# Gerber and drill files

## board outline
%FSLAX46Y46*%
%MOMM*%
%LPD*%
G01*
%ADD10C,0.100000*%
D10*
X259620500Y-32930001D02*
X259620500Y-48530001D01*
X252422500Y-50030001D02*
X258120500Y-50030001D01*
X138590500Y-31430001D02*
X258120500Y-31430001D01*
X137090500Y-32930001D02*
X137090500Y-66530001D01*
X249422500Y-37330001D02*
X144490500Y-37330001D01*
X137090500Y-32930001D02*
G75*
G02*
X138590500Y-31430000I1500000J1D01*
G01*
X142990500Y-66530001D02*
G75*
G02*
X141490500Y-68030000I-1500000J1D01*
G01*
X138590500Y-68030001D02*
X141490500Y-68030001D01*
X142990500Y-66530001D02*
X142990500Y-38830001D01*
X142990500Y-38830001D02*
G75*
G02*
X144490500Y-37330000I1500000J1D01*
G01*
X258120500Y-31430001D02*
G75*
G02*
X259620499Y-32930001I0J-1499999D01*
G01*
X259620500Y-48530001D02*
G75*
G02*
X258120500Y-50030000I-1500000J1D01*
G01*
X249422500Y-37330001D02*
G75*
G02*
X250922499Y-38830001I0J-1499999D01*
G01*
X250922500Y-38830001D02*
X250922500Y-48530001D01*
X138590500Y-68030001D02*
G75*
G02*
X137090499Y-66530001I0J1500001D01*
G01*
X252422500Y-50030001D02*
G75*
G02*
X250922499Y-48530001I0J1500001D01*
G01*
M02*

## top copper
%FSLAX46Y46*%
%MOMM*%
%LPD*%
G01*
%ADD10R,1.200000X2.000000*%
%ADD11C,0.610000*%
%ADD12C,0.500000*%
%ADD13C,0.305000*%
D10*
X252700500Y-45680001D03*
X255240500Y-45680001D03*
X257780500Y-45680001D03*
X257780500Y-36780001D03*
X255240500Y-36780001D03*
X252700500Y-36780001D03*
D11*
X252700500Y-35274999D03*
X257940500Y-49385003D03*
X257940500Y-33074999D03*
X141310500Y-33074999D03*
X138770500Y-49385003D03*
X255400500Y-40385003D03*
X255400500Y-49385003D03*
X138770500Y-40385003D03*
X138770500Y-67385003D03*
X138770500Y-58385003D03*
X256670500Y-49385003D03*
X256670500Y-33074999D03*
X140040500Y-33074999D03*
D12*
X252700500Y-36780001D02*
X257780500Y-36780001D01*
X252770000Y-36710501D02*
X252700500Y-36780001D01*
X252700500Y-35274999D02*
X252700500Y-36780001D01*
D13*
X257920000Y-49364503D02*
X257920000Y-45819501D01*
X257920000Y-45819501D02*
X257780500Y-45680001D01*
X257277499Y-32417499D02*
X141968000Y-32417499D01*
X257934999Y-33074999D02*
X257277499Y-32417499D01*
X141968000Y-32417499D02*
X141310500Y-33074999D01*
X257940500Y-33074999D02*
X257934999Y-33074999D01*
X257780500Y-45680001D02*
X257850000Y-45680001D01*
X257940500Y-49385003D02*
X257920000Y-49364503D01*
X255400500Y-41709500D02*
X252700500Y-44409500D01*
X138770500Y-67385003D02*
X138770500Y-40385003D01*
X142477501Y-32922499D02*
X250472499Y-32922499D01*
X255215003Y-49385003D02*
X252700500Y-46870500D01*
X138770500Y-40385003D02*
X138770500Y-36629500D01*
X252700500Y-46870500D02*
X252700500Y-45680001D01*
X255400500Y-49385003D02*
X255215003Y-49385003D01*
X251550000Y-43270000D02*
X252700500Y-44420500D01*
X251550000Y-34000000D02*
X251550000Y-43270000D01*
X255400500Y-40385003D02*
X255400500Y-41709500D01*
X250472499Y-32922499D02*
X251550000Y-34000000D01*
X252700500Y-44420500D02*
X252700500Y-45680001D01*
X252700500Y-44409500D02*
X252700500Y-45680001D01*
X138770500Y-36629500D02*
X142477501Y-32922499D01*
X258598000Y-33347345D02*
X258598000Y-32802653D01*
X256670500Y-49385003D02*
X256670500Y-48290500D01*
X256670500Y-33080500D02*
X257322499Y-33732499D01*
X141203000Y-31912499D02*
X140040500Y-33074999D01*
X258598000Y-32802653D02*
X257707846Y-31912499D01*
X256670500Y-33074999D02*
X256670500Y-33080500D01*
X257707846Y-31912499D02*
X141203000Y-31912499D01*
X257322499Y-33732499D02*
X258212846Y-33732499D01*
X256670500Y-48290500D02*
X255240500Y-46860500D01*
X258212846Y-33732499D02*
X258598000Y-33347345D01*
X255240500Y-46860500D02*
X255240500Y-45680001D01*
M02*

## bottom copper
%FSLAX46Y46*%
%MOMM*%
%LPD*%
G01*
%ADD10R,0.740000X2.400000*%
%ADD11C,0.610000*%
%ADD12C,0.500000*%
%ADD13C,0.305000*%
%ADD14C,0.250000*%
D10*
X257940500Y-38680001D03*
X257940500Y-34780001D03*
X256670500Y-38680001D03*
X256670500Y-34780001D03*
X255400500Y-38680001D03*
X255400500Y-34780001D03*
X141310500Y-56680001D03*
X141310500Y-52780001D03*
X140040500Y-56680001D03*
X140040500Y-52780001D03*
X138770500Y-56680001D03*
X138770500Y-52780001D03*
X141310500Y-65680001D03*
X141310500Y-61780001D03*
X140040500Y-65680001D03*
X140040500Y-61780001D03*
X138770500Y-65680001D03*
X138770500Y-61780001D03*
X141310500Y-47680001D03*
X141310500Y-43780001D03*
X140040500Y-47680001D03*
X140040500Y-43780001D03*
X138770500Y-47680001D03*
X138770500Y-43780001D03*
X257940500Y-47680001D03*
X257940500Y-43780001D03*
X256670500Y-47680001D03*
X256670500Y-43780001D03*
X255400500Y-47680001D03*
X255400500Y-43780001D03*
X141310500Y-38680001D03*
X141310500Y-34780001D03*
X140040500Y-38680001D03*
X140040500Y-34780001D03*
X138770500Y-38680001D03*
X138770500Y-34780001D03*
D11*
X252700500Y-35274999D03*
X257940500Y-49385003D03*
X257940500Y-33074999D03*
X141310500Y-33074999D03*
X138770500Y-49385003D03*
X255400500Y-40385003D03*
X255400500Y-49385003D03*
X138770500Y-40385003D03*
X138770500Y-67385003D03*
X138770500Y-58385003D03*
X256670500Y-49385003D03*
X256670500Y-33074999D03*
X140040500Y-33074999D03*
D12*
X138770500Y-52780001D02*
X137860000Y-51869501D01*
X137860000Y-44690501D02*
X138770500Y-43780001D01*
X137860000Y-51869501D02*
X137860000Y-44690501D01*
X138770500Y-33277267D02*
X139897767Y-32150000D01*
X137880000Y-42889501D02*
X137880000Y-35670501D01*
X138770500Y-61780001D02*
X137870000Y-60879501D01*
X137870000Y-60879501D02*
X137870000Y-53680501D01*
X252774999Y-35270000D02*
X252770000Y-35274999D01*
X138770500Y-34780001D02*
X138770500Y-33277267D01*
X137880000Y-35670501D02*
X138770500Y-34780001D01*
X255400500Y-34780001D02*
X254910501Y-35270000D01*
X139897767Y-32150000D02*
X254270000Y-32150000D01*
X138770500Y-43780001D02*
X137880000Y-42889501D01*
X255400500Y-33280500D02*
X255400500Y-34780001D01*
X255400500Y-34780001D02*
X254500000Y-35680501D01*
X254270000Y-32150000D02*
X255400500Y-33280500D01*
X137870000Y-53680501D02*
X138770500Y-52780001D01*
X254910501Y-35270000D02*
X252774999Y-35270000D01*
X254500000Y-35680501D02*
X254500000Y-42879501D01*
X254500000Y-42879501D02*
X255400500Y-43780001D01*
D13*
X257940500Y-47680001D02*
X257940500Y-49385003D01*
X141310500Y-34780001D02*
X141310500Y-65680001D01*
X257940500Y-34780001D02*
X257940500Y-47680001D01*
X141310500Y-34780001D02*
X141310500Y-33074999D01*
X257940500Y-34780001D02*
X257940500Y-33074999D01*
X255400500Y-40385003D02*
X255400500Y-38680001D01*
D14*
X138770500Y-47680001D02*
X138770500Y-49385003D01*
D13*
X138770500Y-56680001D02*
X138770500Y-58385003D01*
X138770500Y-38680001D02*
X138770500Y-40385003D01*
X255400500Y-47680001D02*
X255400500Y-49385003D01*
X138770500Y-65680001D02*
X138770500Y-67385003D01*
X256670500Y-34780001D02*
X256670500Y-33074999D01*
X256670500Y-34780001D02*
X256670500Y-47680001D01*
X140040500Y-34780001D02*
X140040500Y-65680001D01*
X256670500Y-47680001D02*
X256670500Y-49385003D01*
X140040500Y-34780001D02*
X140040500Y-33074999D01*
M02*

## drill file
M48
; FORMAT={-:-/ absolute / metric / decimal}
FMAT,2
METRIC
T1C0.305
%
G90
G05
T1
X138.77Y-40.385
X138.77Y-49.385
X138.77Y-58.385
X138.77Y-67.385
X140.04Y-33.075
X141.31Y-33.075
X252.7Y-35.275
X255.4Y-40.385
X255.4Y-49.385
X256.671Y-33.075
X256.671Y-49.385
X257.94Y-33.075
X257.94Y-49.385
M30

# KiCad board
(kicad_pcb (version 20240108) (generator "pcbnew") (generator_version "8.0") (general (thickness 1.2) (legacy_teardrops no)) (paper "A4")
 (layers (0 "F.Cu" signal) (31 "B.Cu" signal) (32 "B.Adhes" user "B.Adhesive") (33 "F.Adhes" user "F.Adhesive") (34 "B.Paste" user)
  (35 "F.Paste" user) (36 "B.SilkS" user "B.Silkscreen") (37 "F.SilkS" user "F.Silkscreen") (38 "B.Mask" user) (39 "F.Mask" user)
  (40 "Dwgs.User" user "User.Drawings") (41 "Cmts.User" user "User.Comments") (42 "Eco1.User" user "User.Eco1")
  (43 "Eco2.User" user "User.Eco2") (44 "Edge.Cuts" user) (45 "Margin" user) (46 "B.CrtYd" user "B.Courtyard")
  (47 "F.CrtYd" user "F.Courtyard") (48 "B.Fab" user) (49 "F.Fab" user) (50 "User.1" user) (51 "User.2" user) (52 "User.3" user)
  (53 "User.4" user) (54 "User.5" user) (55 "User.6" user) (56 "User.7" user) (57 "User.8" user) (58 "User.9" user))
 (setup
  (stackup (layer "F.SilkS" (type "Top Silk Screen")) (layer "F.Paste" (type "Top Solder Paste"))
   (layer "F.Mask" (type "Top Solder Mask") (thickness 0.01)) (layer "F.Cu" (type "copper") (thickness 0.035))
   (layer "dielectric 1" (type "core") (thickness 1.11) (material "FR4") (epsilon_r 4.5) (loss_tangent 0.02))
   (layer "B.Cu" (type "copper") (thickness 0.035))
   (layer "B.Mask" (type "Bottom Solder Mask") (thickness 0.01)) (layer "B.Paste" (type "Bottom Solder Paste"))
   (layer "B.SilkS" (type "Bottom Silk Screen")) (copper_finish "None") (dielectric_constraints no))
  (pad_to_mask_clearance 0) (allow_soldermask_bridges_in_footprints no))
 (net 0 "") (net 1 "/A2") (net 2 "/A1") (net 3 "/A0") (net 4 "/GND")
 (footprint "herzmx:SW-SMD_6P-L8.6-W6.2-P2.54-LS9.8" (layer "F.Cu") (at 255.2405 41.230001)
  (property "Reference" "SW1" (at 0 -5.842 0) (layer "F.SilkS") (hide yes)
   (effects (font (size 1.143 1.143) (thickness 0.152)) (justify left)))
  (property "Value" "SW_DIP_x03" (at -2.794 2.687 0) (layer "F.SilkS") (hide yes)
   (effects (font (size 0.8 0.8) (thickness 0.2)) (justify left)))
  (pad "1" smd rect (at -2.54 4.45) (size 1.2 2) (layers "F.Cu" "F.Paste" "F.Mask") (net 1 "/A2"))
  (pad "2" smd rect (at 0 4.45) (size 1.2 2) (layers "F.Cu" "F.Paste" "F.Mask") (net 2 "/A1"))
  (pad "3" smd rect (at 2.54 4.45) (size 1.2 2) (layers "F.Cu" "F.Paste" "F.Mask") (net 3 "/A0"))
  (pad "4" smd rect (at 2.54 -4.45) (size 1.2 2) (layers "F.Cu" "F.Paste" "F.Mask") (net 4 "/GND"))
  (pad "5" smd rect (at 0 -4.45) (size 1.2 2) (layers "F.Cu" "F.Paste" "F.Mask") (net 4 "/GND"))
  (pad "6" smd rect (at -2.54 -4.45) (size 1.2 2) (layers "F.Cu" "F.Paste" "F.Mask") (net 4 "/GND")))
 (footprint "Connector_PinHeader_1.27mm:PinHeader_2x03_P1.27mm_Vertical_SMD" (layer "B.Cu") (at 256.6705 36.730001 90)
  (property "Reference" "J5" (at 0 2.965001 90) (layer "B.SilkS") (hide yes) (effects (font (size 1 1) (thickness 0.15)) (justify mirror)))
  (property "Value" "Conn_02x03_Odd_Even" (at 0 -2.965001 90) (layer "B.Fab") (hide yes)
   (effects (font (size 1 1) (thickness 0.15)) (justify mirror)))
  (pad "1" smd rect (at -1.95 1.27 90) (size 2.4 0.74) (layers "B.Cu" "B.Paste" "B.Mask") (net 3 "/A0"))
  (pad "2" smd rect (at 1.95 1.27 90) (size 2.4 0.74) (layers "B.Cu" "B.Paste" "B.Mask") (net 3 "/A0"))
  (pad "3" smd rect (at -1.95 0 90) (size 2.4 0.74) (layers "B.Cu" "B.Paste" "B.Mask") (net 2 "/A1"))
  (pad "4" smd rect (at 1.95 0 90) (size 2.4 0.74) (layers "B.Cu" "B.Paste" "B.Mask") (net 2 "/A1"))
  (pad "5" smd rect (at -1.95 -1.27 90) (size 2.4 0.74) (layers "B.Cu" "B.Paste" "B.Mask") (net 1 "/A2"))
  (pad "6" smd rect (at 1.95 -1.27 90) (size 2.4 0.74) (layers "B.Cu" "B.Paste" "B.Mask") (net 4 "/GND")))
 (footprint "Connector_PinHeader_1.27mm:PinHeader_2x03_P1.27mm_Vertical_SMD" (layer "B.Cu") (at 140.0405 54.730001 90)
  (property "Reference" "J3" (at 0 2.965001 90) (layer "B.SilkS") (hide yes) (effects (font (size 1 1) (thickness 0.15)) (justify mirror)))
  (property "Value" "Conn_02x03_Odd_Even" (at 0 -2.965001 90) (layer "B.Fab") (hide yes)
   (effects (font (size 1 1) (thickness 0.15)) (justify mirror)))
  (pad "1" smd rect (at -1.95 1.27 90) (size 2.4 0.74) (layers "B.Cu" "B.Paste" "B.Mask") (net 3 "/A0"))
  (pad "2" smd rect (at 1.95 1.27 90) (size 2.4 0.74) (layers "B.Cu" "B.Paste" "B.Mask") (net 3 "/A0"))
  (pad "3" smd rect (at -1.95 0 90) (size 2.4 0.74) (layers "B.Cu" "B.Paste" "B.Mask") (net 2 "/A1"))
  (pad "4" smd rect (at 1.95 0 90) (size 2.4 0.74) (layers "B.Cu" "B.Paste" "B.Mask") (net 2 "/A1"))
  (pad "5" smd rect (at -1.95 -1.27 90) (size 2.4 0.74) (layers "B.Cu" "B.Paste" "B.Mask") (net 1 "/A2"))
  (pad "6" smd rect (at 1.95 -1.27 90) (size 2.4 0.74) (layers "B.Cu" "B.Paste" "B.Mask") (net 4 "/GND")))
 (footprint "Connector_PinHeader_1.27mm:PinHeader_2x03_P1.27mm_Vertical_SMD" (layer "B.Cu") (at 140.0405 63.730001 90)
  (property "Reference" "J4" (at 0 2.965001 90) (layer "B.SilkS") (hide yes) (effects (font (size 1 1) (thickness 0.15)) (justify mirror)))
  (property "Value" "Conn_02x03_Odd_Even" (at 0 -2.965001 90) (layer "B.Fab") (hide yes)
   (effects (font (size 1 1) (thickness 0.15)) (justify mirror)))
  (pad "1" smd rect (at -1.95 1.27 90) (size 2.4 0.74) (layers "B.Cu" "B.Paste" "B.Mask") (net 3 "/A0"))
  (pad "2" smd rect (at 1.95 1.27 90) (size 2.4 0.74) (layers "B.Cu" "B.Paste" "B.Mask") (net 3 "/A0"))
  (pad "3" smd rect (at -1.95 0 90) (size 2.4 0.74) (layers "B.Cu" "B.Paste" "B.Mask") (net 2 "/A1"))
  (pad "4" smd rect (at 1.95 0 90) (size 2.4 0.74) (layers "B.Cu" "B.Paste" "B.Mask") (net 2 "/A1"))
  (pad "5" smd rect (at -1.95 -1.27 90) (size 2.4 0.74) (layers "B.Cu" "B.Paste" "B.Mask") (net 1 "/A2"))
  (pad "6" smd rect (at 1.95 -1.27 90) (size 2.4 0.74) (layers "B.Cu" "B.Paste" "B.Mask") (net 4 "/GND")))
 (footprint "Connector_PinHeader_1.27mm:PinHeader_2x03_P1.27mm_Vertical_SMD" (layer "B.Cu") (at 140.0405 45.730001 90)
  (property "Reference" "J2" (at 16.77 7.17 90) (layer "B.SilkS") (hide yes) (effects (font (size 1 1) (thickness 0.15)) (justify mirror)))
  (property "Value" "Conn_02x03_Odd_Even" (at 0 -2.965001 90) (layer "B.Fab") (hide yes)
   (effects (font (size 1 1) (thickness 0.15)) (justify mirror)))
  (pad "1" smd rect (at -1.95 1.27 90) (size 2.4 0.74) (layers "B.Cu" "B.Paste" "B.Mask") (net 3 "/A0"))
  (pad "2" smd rect (at 1.95 1.27 90) (size 2.4 0.74) (layers "B.Cu" "B.Paste" "B.Mask") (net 3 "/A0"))
  (pad "3" smd rect (at -1.95 0 90) (size 2.4 0.74) (layers "B.Cu" "B.Paste" "B.Mask") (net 2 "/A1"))
  (pad "4" smd rect (at 1.95 0 90) (size 2.4 0.74) (layers "B.Cu" "B.Paste" "B.Mask") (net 2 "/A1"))
  (pad "5" smd rect (at -1.95 -1.27 90) (size 2.4 0.74) (layers "B.Cu" "B.Paste" "B.Mask") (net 1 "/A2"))
  (pad "6" smd rect (at 1.95 -1.27 90) (size 2.4 0.74) (layers "B.Cu" "B.Paste" "B.Mask") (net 4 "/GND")))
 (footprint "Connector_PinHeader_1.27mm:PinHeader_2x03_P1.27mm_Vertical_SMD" (layer "B.Cu") (at 256.6705 45.730001 90)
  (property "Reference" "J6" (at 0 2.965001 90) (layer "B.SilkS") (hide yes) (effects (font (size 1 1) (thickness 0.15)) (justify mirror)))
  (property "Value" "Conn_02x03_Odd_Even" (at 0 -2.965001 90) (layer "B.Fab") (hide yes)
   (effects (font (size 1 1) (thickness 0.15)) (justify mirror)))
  (pad "1" smd rect (at -1.95 1.27 90) (size 2.4 0.74) (layers "B.Cu" "B.Paste" "B.Mask") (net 3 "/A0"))
  (pad "2" smd rect (at 1.95 1.27 90) (size 2.4 0.74) (layers "B.Cu" "B.Paste" "B.Mask") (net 3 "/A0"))
  (pad "3" smd rect (at -1.95 0 90) (size 2.4 0.74) (layers "B.Cu" "B.Paste" "B.Mask") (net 2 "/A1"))
  (pad "4" smd rect (at 1.95 0 90) (size 2.4 0.74) (layers "B.Cu" "B.Paste" "B.Mask") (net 2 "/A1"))
  (pad "5" smd rect (at -1.95 -1.27 90) (size 2.4 0.74) (layers "B.Cu" "B.Paste" "B.Mask") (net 1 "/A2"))
  (pad "6" smd rect (at 1.95 -1.27 90) (size 2.4 0.74) (layers "B.Cu" "B.Paste" "B.Mask") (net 4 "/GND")))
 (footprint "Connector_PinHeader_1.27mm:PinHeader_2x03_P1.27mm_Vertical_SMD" (layer "B.Cu") (at 140.0405 36.730001 90)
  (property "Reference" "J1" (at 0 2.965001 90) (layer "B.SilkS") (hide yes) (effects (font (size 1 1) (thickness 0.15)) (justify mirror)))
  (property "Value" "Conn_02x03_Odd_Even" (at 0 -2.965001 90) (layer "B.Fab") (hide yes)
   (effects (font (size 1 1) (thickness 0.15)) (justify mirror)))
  (pad "1" smd rect (at -1.95 1.27 90) (size 2.4 0.74) (layers "B.Cu" "B.Paste" "B.Mask") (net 3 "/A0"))
  (pad "2" smd rect (at 1.95 1.27 90) (size 2.4 0.74) (layers "B.Cu" "B.Paste" "B.Mask") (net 3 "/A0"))
  (pad "3" smd rect (at -1.95 0 90) (size 2.4 0.74) (layers "B.Cu" "B.Paste" "B.Mask") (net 2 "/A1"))
  (pad "4" smd rect (at 1.95 0 90) (size 2.4 0.74) (layers "B.Cu" "B.Paste" "B.Mask") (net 2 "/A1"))
  (pad "5" smd rect (at -1.95 -1.27 90) (size 2.4 0.74) (layers "B.Cu" "B.Paste" "B.Mask") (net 1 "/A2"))
  (pad "6" smd rect (at 1.95 -1.27 90) (size 2.4 0.74) (layers "B.Cu" "B.Paste" "B.Mask") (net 4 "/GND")))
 (gr_line (start 259.6205 32.930001) (end 259.6205 48.530001) (stroke (width 0.1) (type default)) (layer "Edge.Cuts"))
 (gr_line (start 252.4225 50.030001) (end 258.1205 50.030001) (stroke (width 0.1) (type default)) (layer "Edge.Cuts"))
 (gr_line (start 138.5905 31.430001) (end 258.1205 31.430001) (stroke (width 0.1) (type default)) (layer "Edge.Cuts"))
 (gr_line (start 137.0905 32.930001) (end 137.0905 66.530001) (stroke (width 0.1) (type default)) (layer "Edge.Cuts"))
 (gr_line (start 249.4225 37.330001) (end 144.4905 37.330001) (stroke (width 0.1) (type default)) (layer "Edge.Cuts"))
 (gr_arc (start 137.0905 32.930001) (mid 137.52984 31.869341) (end 138.5905 31.430001) (stroke (width 0.1) (type default))
  (layer "Edge.Cuts"))
 (gr_arc (start 142.9905 66.530001) (mid 142.55116 67.590661) (end 141.4905 68.030001) (stroke (width 0.1) (type default))
  (layer "Edge.Cuts"))
 (gr_line (start 138.5905 68.030001) (end 141.4905 68.030001) (stroke (width 0.1) (type default)) (layer "Edge.Cuts"))
 (gr_line (start 142.9905 66.530001) (end 142.9905 38.830001) (stroke (width 0.1) (type default)) (layer "Edge.Cuts"))
 (gr_arc (start 142.9905 38.830001) (mid 143.429839 37.76934) (end 144.4905 37.330001) (stroke (width 0.1) (type default))
  (layer "Edge.Cuts"))
 (gr_arc (start 258.1205 31.430001) (mid 259.18116 31.869341) (end 259.6205 32.930001) (stroke (width 0.1) (type default))
  (layer "Edge.Cuts"))
 (gr_arc (start 259.6205 48.530001) (mid 259.18116 49.590661) (end 258.1205 50.030001) (stroke (width 0.1) (type default))
  (layer "Edge.Cuts"))
 (gr_arc (start 249.4225 37.330001) (mid 250.48316 37.769341) (end 250.9225 38.830001) (stroke (width 0.1) (type default))
  (layer "Edge.Cuts"))
 (gr_line (start 250.9225 38.830001) (end 250.9225 48.530001) (stroke (width 0.1) (type default)) (layer "Edge.Cuts"))
 (gr_arc (start 138.5905 68.030001) (mid 137.529839 67.590662) (end 137.0905 66.530001) (stroke (width 0.1) (type default))
  (layer "Edge.Cuts"))
 (gr_arc (start 252.4225 50.030001) (mid 251.361839 49.590662) (end 250.9225 48.530001) (stroke (width 0.1) (type default))
  (layer "Edge.Cuts"))
 (segment (start 252.7005 36.780001) (end 257.7805 36.780001) (width 0.5) (layer "F.Cu") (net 4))
 (segment (start 252.77 36.710501) (end 252.7005 36.780001) (width 0.5) (layer "F.Cu") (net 4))
 (segment (start 252.7005 35.274999) (end 252.7005 36.780001) (width 0.5) (layer "F.Cu") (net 4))
 (via (at 252.7005 35.274999) (size 0.61) (drill 0.305) (layers "F.Cu" "B.Cu") (free yes) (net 4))
 (segment (start 138.7705 52.780001) (end 137.86 51.869501) (width 0.5) (layer "B.Cu") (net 4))
 (segment (start 137.86 44.690501) (end 138.7705 43.780001) (width 0.5) (layer "B.Cu") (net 4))
 (segment (start 137.86 51.869501) (end 137.86 44.690501) (width 0.5) (layer "B.Cu") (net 4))
 (segment (start 138.7705 33.277267) (end 139.897767 32.15) (width 0.5) (layer "B.Cu") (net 4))
 (segment (start 137.88 42.889501) (end 137.88 35.670501) (width 0.5) (layer "B.Cu") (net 4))
 (segment (start 138.7705 61.780001) (end 137.87 60.879501) (width 0.5) (layer "B.Cu") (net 4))
 (segment (start 137.87 60.879501) (end 137.87 53.680501) (width 0.5) (layer "B.Cu") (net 4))
 (segment (start 252.774999 35.27) (end 252.77 35.274999) (width 0.5) (layer "B.Cu") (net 4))
 (segment (start 138.7705 34.780001) (end 138.7705 33.277267) (width 0.5) (layer "B.Cu") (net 4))
 (segment (start 137.88 35.670501) (end 138.7705 34.780001) (width 0.5) (layer "B.Cu") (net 4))
 (segment (start 255.4005 34.780001) (end 254.910501 35.27) (width 0.5) (layer "B.Cu") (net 4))
 (segment (start 139.897767 32.15) (end 254.27 32.15) (width 0.5) (layer "B.Cu") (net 4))
 (segment (start 138.7705 43.780001) (end 137.88 42.889501) (width 0.5) (layer "B.Cu") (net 4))
 (segment (start 255.4005 33.2805) (end 255.4005 34.780001) (width 0.5) (layer "B.Cu") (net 4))
 (segment (start 255.4005 34.780001) (end 254.5 35.680501) (width 0.5) (layer "B.Cu") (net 4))
 (segment (start 254.27 32.15) (end 255.4005 33.2805) (width 0.5) (layer "B.Cu") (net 4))
 (segment (start 137.87 53.680501) (end 138.7705 52.780001) (width 0.5) (layer "B.Cu") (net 4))
 (segment (start 254.910501 35.27) (end 252.774999 35.27) (width 0.5) (layer "B.Cu") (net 4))
 (segment (start 254.5 35.680501) (end 254.5 42.879501) (width 0.5) (layer "B.Cu") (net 4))
 (segment (start 254.5 42.879501) (end 255.4005 43.780001) (width 0.5) (layer "B.Cu") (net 4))
 (segment (start 257.92 49.364503) (end 257.92 45.819501) (width 0.305) (layer "F.Cu") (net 3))
 (segment (start 257.92 45.819501) (end 257.7805 45.680001) (width 0.305) (layer "F.Cu") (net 3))
 (segment (start 257.277499 32.417499) (end 141.968 32.417499) (width 0.305) (layer "F.Cu") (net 3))
 (segment (start 257.934999 33.074999) (end 257.277499 32.417499) (width 0.305) (layer "F.Cu") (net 3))
 (segment (start 141.968 32.417499) (end 141.3105 33.074999) (width 0.305) (layer "F.Cu") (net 3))
 (segment (start 257.9405 33.074999) (end 257.934999 33.074999) (width 0.305) (layer "F.Cu") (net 3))
 (segment (start 257.7805 45.680001) (end 257.85 45.680001) (width 0.305) (layer "F.Cu") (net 3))
 (segment (start 257.9405 49.385003) (end 257.92 49.364503) (width 0.305) (layer "F.Cu") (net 3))
 (via (at 257.9405 49.385003) (size 0.61) (drill 0.305) (layers "F.Cu" "B.Cu") (free yes) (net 3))
 (via (at 257.9405 33.074999) (size 0.61) (drill 0.305) (layers "F.Cu" "B.Cu") (free yes) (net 3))
 (via (at 141.3105 33.074999) (size 0.61) (drill 0.305) (layers "F.Cu" "B.Cu") (free yes) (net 3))
 (segment (start 257.9405 47.680001) (end 257.9405 49.385003) (width 0.305) (layer "B.Cu") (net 3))
 (segment (start 141.3105 34.780001) (end 141.3105 65.680001) (width 0.305) (layer "B.Cu") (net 3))
 (segment (start 257.9405 34.780001) (end 257.9405 47.680001) (width 0.305) (layer "B.Cu") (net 3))
 (segment (start 141.3105 34.780001) (end 141.3105 33.074999) (width 0.305) (layer "B.Cu") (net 3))
 (segment (start 257.9405 34.780001) (end 257.9405 33.074999) (width 0.305) (layer "B.Cu") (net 3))
 (segment (start 255.4005 41.7095) (end 252.7005 44.4095) (width 0.305) (layer "F.Cu") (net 1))
 (segment (start 138.7705 67.385003) (end 138.7705 40.385003) (width 0.305) (layer "F.Cu") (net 1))
 (segment (start 142.477501 32.922499) (end 250.472499 32.922499) (width 0.305) (layer "F.Cu") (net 1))
 (segment (start 255.215003 49.385003) (end 252.7005 46.8705) (width 0.305) (layer "F.Cu") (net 1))
 (segment (start 138.7705 40.385003) (end 138.7705 36.6295) (width 0.305) (layer "F.Cu") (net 1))
 (segment (start 252.7005 46.8705) (end 252.7005 45.680001) (width 0.305) (layer "F.Cu") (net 1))
 (segment (start 255.4005 49.385003) (end 255.215003 49.385003) (width 0.305) (layer "F.Cu") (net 1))
 (segment (start 251.55 43.27) (end 252.7005 44.4205) (width 0.305) (layer "F.Cu") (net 1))
 (segment (start 251.55 34) (end 251.55 43.27) (width 0.305) (layer "F.Cu") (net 1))
 (segment (start 255.4005 40.385003) (end 255.4005 41.7095) (width 0.305) (layer "F.Cu") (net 1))
 (segment (start 250.472499 32.922499) (end 251.55 34) (width 0.305) (layer "F.Cu") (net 1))
 (segment (start 252.7005 44.4205) (end 252.7005 45.680001) (width 0.305) (layer "F.Cu") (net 1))
 (segment (start 252.7005 44.4095) (end 252.7005 45.680001) (width 0.305) (layer "F.Cu") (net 1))
 (segment (start 138.7705 36.6295) (end 142.477501 32.922499) (width 0.305) (layer "F.Cu") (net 1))
 (via (at 138.7705 49.385003) (size 0.61) (drill 0.305) (layers "F.Cu" "B.Cu") (free yes) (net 1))
 (via (at 255.4005 40.385003) (size 0.61) (drill 0.305) (layers "F.Cu" "B.Cu") (free yes) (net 1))
 (via (at 255.4005 49.385003) (size 0.61) (drill 0.305) (layers "F.Cu" "B.Cu") (free yes) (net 1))
 (via (at 138.7705 40.385003) (size 0.61) (drill 0.305) (layers "F.Cu" "B.Cu") (free yes) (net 1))
 (via (at 138.7705 67.385003) (size 0.61) (drill 0.305) (layers "F.Cu" "B.Cu") (free yes) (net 1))
 (via (at 138.7705 58.385003) (size 0.61) (drill 0.305) (layers "F.Cu" "B.Cu") (free yes) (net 1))
 (segment (start 255.4005 40.385003) (end 255.4005 38.680001) (width 0.305) (layer "B.Cu") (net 1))
 (segment (start 138.7705 47.680001) (end 138.7705 49.385003) (width 0.25) (layer "B.Cu") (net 1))
 (segment (start 138.7705 56.680001) (end 138.7705 58.385003) (width 0.305) (layer "B.Cu") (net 1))
 (segment (start 138.7705 38.680001) (end 138.7705 40.385003) (width 0.305) (layer "B.Cu") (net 1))
 (segment (start 255.4005 47.680001) (end 255.4005 49.385003) (width 0.305) (layer "B.Cu") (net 1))
 (segment (start 138.7705 65.680001) (end 138.7705 67.385003) (width 0.305) (layer "B.Cu") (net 1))
 (segment (start 258.598 33.347345) (end 258.598 32.802653) (width 0.305) (layer "F.Cu") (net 2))
 (segment (start 256.6705 49.385003) (end 256.6705 48.2905) (width 0.305) (layer "F.Cu") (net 2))
 (segment (start 256.6705 33.0805) (end 257.322499 33.732499) (width 0.305) (layer "F.Cu") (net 2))
 (segment (start 141.203 31.912499) (end 140.0405 33.074999) (width 0.305) (layer "F.Cu") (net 2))
 (segment (start 258.598 32.802653) (end 257.707846 31.912499) (width 0.305) (layer "F.Cu") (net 2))
 (segment (start 256.6705 33.074999) (end 256.6705 33.0805) (width 0.305) (layer "F.Cu") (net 2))
 (segment (start 257.707846 31.912499) (end 141.203 31.912499) (width 0.305) (layer "F.Cu") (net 2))
 (segment (start 257.322499 33.732499) (end 258.212846 33.732499) (width 0.305) (layer "F.Cu") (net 2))
 (segment (start 256.6705 48.2905) (end 255.2405 46.8605) (width 0.305) (layer "F.Cu") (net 2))
 (segment (start 258.212846 33.732499) (end 258.598 33.347345) (width 0.305) (layer "F.Cu") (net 2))
 (segment (start 255.2405 46.8605) (end 255.2405 45.680001) (width 0.305) (layer "F.Cu") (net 2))
 (via (at 256.6705 49.385003) (size 0.61) (drill 0.305) (layers "F.Cu" "B.Cu") (free yes) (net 2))
 (via (at 256.6705 33.074999) (size 0.61) (drill 0.305) (layers "F.Cu" "B.Cu") (free yes) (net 2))
 (via (at 140.0405 33.074999) (size 0.61) (drill 0.305) (layers "F.Cu" "B.Cu") (free yes) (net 2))
 (segment (start 256.6705 34.780001) (end 256.6705 33.074999) (width 0.305) (layer "B.Cu") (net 2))
 (segment (start 256.6705 34.780001) (end 256.6705 47.680001) (width 0.305) (layer "B.Cu") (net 2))
 (segment (start 140.0405 34.780001) (end 140.0405 65.680001) (width 0.305) (layer "B.Cu") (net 2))
 (segment (start 256.6705 47.680001) (end 256.6705 49.385003) (width 0.305) (layer "B.Cu") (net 2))
 (segment (start 140.0405 34.780001) (end 140.0405 33.074999) (width 0.305) (layer "B.Cu") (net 2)))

